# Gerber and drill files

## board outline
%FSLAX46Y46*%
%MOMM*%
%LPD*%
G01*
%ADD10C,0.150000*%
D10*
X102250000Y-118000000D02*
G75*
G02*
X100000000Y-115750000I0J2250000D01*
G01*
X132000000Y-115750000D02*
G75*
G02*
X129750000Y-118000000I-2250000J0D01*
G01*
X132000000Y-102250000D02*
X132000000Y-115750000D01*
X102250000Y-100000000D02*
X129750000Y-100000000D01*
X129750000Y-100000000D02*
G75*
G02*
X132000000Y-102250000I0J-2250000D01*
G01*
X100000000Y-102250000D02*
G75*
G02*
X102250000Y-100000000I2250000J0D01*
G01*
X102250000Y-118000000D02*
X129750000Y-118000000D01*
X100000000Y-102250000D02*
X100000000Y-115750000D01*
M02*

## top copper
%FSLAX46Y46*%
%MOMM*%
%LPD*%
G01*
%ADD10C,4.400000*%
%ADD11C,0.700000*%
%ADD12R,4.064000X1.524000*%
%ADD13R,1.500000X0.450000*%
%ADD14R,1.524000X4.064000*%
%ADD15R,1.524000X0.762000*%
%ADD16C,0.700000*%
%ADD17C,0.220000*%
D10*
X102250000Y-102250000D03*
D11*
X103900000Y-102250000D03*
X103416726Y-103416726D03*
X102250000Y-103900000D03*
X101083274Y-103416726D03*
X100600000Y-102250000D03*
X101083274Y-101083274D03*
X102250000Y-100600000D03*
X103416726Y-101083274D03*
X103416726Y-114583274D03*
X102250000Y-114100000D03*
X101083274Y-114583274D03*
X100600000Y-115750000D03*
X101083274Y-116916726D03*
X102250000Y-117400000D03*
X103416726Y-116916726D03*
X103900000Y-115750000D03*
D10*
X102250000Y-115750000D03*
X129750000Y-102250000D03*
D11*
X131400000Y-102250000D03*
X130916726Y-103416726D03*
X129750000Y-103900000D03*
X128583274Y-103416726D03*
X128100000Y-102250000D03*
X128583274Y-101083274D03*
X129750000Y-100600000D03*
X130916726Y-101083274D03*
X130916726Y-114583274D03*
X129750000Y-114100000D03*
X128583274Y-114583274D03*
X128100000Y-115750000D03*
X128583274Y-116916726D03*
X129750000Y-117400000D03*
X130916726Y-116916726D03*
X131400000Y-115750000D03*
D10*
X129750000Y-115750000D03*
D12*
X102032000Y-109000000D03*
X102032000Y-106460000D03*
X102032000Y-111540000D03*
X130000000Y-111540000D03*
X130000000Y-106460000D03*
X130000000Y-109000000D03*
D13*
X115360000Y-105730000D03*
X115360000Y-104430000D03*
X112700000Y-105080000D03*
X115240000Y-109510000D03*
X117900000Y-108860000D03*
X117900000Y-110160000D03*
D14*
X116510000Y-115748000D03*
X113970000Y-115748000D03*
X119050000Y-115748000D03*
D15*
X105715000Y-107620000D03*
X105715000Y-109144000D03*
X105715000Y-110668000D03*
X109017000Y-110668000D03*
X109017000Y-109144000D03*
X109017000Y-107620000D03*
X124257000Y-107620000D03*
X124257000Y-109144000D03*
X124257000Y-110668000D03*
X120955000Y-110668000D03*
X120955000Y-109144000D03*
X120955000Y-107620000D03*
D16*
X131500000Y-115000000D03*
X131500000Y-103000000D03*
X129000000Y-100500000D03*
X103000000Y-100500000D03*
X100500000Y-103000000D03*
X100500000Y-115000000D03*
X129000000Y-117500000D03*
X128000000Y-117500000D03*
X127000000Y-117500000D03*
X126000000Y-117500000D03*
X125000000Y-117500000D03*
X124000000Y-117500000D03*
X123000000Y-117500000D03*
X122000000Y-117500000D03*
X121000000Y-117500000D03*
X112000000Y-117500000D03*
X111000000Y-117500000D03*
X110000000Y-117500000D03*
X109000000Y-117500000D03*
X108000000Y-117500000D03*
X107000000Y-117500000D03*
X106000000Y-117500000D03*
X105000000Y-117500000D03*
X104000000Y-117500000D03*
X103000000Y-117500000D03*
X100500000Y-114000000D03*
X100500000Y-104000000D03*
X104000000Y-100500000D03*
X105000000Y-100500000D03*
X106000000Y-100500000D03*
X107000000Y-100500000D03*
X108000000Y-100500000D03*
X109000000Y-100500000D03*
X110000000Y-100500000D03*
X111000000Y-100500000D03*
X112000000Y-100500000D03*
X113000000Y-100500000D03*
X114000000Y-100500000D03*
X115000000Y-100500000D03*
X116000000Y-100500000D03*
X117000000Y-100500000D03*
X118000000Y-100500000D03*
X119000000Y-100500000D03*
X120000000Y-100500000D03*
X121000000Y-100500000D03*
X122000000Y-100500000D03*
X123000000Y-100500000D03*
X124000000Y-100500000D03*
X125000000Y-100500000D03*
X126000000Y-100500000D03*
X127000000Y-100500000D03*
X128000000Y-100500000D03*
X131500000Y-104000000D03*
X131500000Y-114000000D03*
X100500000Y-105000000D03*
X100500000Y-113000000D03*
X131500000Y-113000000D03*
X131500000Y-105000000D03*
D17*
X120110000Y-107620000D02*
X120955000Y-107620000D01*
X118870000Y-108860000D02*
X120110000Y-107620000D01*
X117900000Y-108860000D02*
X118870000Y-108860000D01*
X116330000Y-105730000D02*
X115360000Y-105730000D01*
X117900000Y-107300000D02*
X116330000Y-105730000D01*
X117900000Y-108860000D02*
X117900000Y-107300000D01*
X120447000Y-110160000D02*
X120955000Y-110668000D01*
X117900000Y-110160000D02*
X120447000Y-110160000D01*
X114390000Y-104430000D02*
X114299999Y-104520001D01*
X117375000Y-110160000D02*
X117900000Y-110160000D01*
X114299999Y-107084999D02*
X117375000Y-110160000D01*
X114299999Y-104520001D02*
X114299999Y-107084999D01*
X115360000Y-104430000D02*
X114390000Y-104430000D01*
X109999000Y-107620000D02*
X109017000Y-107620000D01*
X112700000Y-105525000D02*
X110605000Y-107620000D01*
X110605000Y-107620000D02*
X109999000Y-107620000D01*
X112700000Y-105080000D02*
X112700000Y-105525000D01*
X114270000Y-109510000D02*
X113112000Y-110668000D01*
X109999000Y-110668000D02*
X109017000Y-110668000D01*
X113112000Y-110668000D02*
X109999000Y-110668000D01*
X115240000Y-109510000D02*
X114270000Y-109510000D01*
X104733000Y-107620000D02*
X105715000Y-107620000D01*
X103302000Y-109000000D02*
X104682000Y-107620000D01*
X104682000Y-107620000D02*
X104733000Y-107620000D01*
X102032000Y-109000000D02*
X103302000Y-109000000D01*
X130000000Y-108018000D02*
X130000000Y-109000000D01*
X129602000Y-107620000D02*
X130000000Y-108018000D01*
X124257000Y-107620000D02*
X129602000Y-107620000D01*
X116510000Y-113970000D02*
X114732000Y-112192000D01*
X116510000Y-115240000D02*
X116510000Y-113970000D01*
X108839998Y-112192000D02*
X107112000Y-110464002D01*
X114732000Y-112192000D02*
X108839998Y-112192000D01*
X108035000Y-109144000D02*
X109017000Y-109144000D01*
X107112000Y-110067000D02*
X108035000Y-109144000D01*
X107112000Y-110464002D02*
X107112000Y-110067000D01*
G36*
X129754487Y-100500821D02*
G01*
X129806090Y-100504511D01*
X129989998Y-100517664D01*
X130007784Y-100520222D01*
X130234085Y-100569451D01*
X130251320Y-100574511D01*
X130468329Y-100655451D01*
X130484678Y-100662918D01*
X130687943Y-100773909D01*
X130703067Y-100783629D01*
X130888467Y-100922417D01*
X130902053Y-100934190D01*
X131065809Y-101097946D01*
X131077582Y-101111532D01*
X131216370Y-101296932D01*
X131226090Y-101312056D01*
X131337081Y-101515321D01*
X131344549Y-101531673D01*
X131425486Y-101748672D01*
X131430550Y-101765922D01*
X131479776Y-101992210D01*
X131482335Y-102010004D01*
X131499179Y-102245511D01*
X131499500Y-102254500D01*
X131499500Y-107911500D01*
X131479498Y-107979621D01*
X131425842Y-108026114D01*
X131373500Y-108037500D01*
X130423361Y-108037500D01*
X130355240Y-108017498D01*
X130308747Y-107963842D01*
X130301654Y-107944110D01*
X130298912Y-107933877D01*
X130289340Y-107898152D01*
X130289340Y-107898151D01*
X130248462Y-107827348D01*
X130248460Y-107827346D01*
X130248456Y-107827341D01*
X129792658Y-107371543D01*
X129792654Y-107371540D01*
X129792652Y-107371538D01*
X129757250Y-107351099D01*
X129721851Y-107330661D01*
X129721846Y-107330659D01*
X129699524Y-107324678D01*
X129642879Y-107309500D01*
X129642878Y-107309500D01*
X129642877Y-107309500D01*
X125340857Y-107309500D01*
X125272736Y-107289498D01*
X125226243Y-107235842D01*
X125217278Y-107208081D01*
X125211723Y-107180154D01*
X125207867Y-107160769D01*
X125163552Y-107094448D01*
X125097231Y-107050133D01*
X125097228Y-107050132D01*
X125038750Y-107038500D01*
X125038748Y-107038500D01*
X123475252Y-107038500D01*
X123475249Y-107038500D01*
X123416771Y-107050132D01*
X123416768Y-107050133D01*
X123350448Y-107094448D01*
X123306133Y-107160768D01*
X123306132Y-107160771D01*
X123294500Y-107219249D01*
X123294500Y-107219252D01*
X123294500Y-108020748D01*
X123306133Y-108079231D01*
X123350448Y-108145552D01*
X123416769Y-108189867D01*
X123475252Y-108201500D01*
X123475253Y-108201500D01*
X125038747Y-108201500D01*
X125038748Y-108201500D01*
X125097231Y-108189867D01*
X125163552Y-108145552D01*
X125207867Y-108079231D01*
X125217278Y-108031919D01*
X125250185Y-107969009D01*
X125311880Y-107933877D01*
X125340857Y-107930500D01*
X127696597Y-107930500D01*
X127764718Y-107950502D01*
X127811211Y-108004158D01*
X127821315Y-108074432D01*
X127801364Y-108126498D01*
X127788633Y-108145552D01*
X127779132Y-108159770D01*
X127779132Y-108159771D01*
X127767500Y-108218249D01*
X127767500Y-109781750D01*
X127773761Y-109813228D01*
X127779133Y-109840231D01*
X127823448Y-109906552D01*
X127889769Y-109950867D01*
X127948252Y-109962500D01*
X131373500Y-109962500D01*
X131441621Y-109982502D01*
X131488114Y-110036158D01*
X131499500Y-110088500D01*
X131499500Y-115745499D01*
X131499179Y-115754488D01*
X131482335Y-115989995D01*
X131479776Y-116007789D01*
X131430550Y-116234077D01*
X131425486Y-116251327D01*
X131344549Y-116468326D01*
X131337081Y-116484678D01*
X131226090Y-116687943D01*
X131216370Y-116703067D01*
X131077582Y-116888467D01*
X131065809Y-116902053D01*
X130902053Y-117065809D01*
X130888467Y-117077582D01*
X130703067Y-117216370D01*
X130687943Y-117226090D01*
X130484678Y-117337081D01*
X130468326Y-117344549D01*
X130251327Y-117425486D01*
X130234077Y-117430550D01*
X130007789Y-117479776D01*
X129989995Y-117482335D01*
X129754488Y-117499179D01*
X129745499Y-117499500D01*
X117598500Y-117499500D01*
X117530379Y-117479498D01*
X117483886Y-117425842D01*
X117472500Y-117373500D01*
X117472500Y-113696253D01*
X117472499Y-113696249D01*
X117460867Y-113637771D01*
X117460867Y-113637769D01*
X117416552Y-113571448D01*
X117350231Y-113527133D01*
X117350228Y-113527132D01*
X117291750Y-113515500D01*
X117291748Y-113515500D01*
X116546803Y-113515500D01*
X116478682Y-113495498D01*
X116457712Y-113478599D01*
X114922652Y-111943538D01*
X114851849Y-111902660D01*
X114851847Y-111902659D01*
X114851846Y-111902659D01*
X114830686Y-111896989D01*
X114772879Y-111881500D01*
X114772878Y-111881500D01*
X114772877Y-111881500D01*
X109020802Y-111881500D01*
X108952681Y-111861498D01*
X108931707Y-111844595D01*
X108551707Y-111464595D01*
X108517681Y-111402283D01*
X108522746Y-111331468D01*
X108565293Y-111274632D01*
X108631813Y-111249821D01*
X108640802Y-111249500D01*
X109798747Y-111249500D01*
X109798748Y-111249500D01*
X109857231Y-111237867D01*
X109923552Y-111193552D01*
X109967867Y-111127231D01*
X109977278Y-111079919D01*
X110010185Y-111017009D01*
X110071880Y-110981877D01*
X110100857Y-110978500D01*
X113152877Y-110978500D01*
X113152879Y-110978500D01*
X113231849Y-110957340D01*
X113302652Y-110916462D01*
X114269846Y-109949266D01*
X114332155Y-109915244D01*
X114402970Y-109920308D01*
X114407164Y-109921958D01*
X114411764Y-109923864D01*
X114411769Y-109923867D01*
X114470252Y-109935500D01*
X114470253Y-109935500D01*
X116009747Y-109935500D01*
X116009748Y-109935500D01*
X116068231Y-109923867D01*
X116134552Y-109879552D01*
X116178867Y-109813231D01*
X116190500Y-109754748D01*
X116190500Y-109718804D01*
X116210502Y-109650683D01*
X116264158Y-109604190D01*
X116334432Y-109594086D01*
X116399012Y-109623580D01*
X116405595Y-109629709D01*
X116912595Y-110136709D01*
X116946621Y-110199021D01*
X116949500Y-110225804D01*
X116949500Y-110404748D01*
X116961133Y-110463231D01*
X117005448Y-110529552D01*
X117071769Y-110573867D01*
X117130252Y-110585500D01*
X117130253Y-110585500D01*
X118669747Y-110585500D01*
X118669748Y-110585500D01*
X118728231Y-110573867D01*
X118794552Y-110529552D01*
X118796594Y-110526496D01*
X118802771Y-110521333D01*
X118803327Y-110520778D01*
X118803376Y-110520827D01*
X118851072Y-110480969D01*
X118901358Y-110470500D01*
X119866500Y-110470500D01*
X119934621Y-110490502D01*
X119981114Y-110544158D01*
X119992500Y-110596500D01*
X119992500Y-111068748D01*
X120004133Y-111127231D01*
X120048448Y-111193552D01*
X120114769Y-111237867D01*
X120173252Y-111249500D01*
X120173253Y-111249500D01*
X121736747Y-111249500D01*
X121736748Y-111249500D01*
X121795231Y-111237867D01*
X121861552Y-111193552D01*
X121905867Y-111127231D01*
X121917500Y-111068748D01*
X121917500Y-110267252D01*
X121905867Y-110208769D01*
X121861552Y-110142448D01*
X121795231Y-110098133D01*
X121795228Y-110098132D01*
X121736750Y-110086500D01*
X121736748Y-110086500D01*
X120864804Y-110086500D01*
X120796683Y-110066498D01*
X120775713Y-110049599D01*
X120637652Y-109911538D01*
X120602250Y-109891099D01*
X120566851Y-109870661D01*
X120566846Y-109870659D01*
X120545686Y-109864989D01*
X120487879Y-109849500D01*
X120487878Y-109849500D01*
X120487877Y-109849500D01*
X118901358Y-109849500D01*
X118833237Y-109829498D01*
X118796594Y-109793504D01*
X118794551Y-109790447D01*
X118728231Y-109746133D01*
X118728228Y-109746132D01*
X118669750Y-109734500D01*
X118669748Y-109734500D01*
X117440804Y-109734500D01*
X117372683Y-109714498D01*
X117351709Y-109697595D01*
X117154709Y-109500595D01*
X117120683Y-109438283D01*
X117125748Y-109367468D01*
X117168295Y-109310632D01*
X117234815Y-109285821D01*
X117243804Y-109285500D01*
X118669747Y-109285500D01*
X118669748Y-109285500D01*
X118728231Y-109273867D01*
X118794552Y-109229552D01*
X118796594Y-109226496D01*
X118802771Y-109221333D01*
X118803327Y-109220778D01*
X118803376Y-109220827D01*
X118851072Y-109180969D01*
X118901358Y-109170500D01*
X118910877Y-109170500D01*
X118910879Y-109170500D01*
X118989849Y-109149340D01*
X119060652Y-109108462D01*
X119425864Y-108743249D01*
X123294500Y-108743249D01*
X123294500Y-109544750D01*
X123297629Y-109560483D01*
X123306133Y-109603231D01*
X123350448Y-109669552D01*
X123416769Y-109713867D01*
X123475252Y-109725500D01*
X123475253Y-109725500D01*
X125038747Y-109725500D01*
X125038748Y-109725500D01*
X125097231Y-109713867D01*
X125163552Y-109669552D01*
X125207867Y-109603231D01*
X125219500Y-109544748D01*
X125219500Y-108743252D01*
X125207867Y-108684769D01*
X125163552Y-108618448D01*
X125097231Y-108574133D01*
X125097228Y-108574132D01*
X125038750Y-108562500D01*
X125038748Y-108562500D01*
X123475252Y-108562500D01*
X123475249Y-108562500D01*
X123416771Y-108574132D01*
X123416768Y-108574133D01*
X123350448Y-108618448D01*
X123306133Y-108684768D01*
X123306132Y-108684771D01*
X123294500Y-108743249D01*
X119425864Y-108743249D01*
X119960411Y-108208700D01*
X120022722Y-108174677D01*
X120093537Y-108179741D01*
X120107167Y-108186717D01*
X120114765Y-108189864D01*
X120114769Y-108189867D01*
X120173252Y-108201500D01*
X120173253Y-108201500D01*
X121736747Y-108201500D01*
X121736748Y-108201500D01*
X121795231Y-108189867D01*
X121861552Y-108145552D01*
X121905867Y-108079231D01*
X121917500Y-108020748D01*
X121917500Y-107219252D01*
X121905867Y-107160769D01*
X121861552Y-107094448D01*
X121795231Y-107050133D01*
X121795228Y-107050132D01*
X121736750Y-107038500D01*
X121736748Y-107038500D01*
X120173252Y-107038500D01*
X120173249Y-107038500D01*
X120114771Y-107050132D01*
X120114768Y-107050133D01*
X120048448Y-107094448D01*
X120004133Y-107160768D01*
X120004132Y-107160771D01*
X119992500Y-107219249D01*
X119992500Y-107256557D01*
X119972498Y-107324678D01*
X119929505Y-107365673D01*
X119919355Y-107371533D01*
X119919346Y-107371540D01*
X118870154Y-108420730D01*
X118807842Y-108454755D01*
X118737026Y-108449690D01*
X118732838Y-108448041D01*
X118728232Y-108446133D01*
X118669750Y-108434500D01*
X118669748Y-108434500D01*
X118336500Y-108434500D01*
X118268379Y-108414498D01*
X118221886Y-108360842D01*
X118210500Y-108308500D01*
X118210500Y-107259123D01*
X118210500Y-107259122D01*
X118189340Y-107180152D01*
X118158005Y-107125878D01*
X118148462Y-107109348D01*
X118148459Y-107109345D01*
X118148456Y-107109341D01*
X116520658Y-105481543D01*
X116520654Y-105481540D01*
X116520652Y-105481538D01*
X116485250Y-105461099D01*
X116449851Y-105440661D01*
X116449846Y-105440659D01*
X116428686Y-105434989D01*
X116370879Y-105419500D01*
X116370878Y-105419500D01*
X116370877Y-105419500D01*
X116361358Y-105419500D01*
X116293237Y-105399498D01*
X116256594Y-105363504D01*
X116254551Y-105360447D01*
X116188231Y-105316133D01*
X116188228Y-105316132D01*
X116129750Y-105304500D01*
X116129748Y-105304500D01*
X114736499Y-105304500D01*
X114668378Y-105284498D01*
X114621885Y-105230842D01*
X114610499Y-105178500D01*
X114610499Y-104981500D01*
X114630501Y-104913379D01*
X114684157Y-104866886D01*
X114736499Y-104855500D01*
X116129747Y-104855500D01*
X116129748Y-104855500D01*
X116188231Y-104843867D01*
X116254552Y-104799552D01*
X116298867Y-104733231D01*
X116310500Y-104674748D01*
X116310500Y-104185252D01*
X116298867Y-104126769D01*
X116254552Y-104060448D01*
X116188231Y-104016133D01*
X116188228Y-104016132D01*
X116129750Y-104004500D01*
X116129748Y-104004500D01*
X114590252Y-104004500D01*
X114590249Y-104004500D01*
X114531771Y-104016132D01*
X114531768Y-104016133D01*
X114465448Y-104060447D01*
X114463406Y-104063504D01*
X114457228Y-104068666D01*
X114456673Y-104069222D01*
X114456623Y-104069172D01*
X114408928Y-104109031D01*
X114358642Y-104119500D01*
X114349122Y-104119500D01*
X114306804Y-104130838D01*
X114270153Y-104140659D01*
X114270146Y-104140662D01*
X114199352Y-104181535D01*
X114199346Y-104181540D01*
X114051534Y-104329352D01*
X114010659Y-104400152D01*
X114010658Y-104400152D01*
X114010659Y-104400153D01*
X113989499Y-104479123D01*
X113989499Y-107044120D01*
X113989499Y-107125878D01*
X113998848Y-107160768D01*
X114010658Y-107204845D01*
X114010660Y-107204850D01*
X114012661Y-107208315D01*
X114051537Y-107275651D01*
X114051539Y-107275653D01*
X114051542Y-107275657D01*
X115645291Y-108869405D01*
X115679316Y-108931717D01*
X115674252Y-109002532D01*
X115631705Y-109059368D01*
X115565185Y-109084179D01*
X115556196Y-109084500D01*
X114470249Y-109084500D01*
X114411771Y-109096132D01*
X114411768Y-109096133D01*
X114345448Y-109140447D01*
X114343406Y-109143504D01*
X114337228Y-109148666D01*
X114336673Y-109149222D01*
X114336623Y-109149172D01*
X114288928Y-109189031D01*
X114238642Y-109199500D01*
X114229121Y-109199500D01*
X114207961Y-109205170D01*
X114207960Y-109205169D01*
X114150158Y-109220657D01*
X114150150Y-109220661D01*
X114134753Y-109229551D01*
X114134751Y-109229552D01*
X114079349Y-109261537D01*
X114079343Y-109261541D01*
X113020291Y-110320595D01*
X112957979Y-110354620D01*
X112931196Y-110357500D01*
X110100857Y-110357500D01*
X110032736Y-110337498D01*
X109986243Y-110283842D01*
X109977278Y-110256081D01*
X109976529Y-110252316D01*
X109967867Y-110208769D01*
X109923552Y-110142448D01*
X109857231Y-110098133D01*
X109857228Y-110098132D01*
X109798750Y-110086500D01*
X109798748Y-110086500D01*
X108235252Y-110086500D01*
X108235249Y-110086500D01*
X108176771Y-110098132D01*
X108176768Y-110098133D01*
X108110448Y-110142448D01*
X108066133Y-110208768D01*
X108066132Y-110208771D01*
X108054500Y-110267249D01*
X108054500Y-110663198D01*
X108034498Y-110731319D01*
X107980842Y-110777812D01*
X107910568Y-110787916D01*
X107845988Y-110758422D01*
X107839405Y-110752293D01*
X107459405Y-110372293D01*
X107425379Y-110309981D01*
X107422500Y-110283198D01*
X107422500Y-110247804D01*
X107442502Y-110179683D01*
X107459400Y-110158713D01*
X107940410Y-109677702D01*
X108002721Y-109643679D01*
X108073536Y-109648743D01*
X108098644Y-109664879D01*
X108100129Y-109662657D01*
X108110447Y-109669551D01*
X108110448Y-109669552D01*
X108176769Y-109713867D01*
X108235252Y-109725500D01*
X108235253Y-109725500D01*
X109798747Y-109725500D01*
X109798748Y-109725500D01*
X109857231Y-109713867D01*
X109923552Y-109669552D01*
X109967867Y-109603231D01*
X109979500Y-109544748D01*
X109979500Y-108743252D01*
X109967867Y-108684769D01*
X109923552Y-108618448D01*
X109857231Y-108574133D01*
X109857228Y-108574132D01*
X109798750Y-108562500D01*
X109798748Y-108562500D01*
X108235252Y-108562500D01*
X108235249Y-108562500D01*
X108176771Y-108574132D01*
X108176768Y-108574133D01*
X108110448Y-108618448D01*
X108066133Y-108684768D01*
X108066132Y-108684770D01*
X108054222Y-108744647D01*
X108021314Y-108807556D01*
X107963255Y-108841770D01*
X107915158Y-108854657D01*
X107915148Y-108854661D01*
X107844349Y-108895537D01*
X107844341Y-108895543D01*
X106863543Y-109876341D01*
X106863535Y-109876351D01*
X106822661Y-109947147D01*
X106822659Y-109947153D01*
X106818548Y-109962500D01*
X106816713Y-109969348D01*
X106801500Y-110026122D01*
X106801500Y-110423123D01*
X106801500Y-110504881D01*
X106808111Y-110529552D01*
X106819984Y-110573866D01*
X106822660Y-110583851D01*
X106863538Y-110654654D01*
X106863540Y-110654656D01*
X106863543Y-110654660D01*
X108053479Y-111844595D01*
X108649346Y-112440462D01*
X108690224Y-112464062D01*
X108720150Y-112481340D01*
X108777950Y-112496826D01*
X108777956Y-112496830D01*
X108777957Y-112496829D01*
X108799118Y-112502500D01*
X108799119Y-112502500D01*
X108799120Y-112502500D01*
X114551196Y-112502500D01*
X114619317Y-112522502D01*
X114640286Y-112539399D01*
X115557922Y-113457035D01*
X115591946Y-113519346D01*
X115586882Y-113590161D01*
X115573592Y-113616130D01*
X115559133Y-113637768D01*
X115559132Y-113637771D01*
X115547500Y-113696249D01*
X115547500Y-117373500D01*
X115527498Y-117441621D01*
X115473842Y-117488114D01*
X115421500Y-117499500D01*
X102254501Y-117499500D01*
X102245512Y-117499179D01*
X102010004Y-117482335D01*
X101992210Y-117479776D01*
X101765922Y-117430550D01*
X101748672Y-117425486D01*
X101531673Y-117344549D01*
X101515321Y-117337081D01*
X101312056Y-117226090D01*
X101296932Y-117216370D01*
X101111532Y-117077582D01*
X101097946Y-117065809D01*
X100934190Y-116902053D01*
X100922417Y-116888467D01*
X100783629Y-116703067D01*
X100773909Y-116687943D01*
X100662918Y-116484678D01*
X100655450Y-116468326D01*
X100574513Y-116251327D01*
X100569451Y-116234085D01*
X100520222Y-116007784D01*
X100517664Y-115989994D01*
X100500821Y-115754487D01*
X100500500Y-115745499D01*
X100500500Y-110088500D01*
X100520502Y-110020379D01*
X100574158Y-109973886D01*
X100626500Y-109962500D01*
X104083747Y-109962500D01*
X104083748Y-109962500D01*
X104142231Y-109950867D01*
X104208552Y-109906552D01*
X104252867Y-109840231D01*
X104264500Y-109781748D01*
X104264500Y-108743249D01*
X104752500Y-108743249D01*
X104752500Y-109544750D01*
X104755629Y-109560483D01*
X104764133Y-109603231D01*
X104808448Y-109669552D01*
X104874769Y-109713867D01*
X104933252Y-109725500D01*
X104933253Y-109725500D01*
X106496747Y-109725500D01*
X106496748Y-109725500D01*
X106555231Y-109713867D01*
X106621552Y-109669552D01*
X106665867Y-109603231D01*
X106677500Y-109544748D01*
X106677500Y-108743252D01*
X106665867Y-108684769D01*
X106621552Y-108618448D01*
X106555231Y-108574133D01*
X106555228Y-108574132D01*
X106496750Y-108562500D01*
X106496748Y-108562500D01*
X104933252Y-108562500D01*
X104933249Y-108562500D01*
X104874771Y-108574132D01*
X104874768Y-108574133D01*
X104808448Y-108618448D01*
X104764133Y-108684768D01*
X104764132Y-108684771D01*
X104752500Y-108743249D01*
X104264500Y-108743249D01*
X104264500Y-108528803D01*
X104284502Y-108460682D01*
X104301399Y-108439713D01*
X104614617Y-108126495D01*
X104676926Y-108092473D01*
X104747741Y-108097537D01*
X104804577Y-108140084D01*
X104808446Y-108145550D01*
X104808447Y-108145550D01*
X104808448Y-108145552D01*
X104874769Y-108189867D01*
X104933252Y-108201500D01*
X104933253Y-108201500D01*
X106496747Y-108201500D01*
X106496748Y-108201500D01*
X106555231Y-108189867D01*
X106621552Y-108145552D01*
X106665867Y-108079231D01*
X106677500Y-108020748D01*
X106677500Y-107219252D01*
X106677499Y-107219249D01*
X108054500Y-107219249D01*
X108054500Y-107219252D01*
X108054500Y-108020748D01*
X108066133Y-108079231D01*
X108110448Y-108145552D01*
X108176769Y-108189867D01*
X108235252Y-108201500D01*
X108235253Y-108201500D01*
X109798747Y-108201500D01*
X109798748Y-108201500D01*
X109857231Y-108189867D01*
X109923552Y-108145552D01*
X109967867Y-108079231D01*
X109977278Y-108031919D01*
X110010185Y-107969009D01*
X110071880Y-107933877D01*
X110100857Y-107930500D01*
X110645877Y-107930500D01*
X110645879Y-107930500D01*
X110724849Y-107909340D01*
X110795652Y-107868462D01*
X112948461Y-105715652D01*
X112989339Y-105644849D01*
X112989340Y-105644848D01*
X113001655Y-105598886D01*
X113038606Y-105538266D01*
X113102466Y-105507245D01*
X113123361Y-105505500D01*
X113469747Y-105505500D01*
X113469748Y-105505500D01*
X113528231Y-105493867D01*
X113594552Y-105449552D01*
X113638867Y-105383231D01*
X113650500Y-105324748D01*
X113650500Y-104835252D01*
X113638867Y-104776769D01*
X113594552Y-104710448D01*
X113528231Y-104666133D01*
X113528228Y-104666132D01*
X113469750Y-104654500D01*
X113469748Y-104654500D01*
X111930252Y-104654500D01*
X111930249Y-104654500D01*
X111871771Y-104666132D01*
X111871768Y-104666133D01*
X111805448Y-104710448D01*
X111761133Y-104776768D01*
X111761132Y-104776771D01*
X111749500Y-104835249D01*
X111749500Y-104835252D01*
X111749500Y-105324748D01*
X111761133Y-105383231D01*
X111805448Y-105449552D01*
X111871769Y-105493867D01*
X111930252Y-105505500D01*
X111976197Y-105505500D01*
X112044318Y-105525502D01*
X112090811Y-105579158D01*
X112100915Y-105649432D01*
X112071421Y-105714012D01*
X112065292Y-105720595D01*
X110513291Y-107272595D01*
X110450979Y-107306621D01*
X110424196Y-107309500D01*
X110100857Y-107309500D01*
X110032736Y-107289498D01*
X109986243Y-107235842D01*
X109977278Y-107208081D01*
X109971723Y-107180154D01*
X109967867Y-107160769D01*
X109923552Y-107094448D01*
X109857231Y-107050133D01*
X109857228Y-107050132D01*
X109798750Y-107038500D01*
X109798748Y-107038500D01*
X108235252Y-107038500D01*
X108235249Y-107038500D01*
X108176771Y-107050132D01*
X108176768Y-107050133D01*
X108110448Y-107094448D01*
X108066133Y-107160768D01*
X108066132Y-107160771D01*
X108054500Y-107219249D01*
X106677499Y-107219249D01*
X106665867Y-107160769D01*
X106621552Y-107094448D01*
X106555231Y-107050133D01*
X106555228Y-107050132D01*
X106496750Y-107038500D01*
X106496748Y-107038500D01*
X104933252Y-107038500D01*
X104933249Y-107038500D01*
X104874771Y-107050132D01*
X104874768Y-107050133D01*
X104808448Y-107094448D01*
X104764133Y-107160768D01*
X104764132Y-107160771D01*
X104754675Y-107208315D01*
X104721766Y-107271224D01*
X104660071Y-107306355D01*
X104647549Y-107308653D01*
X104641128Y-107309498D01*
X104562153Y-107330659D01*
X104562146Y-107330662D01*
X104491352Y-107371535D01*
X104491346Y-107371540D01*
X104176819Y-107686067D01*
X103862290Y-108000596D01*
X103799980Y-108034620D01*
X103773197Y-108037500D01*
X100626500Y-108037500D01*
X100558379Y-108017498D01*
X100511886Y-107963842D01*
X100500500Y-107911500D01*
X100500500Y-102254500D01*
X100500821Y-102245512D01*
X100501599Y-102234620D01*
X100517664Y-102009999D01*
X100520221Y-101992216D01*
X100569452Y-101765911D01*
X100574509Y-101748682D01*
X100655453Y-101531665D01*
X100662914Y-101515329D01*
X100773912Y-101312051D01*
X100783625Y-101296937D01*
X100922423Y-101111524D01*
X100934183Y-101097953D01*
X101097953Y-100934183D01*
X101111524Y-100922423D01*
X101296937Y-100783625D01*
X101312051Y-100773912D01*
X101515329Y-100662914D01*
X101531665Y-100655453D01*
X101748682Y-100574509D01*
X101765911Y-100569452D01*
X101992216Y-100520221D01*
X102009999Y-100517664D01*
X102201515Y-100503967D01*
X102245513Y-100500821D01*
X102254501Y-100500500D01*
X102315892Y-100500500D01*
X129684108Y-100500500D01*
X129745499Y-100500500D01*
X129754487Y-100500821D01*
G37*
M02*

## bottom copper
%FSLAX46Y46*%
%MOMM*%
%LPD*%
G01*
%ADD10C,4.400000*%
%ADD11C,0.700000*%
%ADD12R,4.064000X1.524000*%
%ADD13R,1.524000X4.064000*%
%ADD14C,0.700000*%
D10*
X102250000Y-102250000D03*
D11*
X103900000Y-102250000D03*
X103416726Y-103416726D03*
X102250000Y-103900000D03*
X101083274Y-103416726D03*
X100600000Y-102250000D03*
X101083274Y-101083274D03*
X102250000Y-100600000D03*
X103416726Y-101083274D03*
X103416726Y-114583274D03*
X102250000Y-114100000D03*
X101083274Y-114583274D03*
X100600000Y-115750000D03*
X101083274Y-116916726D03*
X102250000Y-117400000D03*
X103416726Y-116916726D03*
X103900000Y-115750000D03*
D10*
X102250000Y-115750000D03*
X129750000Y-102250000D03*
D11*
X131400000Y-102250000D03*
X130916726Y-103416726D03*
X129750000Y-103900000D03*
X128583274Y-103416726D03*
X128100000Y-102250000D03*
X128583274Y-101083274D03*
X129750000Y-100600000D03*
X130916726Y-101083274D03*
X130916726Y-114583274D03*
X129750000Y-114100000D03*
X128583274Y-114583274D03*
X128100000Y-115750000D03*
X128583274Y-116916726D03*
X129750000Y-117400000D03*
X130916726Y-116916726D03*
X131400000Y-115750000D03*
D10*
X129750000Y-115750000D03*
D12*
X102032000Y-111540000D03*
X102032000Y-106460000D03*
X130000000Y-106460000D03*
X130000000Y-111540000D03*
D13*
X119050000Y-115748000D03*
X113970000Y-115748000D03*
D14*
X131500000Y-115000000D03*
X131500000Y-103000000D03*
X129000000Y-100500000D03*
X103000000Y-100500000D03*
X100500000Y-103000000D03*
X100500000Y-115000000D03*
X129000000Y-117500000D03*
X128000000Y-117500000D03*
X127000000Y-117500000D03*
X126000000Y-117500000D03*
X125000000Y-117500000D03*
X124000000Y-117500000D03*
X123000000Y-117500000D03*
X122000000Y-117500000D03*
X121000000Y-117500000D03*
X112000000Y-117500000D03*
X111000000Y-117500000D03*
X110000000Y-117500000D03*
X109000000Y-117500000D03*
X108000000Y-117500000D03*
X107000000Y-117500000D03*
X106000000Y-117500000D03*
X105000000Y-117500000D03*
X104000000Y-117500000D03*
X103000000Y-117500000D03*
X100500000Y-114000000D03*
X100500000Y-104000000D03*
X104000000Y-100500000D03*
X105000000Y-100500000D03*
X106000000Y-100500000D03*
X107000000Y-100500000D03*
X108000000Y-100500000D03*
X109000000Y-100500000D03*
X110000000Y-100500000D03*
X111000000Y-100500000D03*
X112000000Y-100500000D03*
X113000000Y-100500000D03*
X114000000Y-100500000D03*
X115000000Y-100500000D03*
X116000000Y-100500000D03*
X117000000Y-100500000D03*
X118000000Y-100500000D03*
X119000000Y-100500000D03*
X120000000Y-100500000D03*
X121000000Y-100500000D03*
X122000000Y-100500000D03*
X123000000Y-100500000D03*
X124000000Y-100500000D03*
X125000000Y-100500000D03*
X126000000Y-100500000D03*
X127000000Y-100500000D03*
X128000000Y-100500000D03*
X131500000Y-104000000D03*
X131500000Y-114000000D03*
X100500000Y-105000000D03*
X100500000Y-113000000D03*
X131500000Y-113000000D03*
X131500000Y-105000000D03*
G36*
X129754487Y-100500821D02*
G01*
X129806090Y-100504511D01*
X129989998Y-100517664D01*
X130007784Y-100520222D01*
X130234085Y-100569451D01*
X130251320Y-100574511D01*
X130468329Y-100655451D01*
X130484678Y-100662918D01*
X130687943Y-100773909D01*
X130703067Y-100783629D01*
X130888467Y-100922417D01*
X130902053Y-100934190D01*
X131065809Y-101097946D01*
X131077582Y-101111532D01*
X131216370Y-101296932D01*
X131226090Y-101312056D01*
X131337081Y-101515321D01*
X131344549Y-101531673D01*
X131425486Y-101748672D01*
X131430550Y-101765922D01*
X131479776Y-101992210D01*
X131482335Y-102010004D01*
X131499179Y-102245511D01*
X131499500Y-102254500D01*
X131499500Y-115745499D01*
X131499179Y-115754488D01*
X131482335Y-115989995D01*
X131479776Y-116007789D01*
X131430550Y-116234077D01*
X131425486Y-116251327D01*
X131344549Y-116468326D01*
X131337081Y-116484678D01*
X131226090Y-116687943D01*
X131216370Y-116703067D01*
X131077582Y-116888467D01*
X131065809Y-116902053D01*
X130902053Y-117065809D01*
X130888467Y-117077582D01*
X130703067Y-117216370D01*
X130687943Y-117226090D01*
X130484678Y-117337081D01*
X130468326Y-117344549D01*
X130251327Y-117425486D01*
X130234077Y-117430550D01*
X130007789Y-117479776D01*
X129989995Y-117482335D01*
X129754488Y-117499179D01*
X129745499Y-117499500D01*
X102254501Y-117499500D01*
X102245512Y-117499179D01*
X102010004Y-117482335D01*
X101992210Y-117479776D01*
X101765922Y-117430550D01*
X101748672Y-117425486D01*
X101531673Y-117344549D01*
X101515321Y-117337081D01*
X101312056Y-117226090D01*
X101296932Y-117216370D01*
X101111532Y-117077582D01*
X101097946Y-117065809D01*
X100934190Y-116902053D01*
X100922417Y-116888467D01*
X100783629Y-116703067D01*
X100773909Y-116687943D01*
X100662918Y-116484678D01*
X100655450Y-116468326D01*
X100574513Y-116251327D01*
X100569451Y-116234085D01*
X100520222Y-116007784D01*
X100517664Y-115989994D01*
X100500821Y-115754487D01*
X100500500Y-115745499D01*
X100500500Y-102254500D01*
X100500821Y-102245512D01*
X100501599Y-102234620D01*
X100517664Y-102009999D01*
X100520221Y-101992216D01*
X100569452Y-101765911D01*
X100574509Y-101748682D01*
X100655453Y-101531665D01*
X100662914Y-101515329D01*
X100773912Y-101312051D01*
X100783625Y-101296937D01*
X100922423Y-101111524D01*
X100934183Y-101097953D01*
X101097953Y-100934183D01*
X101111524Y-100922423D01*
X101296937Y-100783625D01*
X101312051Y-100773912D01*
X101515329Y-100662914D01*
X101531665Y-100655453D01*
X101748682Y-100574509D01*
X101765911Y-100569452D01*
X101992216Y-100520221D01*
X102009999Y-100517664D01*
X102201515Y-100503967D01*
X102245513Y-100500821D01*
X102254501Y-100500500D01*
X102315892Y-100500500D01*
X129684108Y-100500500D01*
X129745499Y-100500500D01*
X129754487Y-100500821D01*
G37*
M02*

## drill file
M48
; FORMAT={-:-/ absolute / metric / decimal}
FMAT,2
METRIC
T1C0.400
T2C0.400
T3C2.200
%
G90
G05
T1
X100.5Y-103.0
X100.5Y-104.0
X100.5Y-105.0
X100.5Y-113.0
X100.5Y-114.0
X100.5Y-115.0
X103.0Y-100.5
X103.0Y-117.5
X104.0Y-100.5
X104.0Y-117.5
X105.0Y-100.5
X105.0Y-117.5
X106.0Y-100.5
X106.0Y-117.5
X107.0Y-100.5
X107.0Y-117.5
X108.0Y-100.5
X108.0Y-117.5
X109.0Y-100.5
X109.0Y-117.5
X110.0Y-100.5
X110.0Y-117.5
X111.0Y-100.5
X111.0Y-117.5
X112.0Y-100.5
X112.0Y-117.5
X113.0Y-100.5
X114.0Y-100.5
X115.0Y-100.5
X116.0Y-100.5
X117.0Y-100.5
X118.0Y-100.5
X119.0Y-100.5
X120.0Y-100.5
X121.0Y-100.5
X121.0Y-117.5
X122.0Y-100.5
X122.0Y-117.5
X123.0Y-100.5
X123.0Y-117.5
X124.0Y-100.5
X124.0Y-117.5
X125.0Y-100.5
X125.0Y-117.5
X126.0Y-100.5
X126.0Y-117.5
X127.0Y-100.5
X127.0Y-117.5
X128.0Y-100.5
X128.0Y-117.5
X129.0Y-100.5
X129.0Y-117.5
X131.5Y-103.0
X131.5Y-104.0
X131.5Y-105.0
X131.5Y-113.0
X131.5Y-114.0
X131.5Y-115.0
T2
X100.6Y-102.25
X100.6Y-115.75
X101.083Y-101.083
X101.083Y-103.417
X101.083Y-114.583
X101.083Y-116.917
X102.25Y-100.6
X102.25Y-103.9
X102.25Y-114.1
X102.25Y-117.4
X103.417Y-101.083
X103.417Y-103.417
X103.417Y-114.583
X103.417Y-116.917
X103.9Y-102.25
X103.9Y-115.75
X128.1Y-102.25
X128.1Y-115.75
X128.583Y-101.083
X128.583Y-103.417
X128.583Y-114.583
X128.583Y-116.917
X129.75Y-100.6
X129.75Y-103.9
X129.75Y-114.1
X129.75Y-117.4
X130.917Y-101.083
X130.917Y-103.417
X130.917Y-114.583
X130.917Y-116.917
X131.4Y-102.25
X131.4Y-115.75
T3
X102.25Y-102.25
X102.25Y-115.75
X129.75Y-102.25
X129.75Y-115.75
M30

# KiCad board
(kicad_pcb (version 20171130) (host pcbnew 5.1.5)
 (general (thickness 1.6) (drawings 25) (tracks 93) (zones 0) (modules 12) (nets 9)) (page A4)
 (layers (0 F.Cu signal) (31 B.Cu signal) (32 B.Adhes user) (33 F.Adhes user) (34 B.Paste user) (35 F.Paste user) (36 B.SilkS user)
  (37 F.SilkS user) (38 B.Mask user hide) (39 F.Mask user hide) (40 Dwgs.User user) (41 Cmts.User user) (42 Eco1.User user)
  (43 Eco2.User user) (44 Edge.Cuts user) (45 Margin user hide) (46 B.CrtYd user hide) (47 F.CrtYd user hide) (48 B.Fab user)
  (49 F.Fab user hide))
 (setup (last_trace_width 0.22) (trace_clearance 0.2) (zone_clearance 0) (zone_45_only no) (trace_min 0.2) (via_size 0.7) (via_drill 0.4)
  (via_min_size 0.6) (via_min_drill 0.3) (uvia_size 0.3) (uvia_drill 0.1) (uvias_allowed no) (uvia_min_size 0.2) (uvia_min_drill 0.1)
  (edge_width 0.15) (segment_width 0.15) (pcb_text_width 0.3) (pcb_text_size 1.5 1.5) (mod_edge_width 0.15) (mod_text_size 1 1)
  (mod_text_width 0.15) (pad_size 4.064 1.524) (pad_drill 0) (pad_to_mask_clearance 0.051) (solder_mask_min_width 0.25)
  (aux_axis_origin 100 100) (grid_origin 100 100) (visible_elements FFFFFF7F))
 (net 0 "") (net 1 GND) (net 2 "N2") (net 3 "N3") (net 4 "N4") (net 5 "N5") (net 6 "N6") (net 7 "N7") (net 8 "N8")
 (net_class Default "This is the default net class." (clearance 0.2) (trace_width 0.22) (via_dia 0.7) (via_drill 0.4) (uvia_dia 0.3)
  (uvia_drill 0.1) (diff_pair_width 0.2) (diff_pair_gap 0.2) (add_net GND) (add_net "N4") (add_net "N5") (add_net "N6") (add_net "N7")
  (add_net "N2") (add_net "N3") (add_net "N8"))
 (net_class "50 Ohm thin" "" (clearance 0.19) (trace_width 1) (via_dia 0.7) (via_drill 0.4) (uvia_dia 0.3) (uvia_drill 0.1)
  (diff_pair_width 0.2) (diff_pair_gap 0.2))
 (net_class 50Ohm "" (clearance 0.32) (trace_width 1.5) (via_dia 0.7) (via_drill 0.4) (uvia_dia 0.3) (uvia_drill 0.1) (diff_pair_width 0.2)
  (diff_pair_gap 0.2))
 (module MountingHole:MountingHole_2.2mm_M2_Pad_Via (layer F.Cu) (at 102.25 102.25)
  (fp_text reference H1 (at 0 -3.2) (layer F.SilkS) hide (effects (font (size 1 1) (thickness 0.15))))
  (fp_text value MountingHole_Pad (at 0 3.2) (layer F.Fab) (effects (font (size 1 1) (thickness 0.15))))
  (pad 1 thru_hole circle (at 0 0) (size 4.4 4.4) (drill 2.2) (layers *.Cu *.Mask) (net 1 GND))
  (pad 1 thru_hole circle (at 1.65 0) (size 0.7 0.7) (drill 0.4) (layers *.Cu *.Mask) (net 1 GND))
  (pad 1 thru_hole circle (at 1.166726 1.166726) (size 0.7 0.7) (drill 0.4) (layers *.Cu *.Mask) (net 1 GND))
  (pad 1 thru_hole circle (at 0 1.65) (size 0.7 0.7) (drill 0.4) (layers *.Cu *.Mask) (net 1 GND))
  (pad 1 thru_hole circle (at -1.166726 1.166726) (size 0.7 0.7) (drill 0.4) (layers *.Cu *.Mask) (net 1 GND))
  (pad 1 thru_hole circle (at -1.65 0) (size 0.7 0.7) (drill 0.4) (layers *.Cu *.Mask) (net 1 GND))
  (pad 1 thru_hole circle (at -1.166726 -1.166726) (size 0.7 0.7) (drill 0.4) (layers *.Cu *.Mask) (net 1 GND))
  (pad 1 thru_hole circle (at 0 -1.65) (size 0.7 0.7) (drill 0.4) (layers *.Cu *.Mask) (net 1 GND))
  (pad 1 thru_hole circle (at 1.166726 -1.166726) (size 0.7 0.7) (drill 0.4) (layers *.Cu *.Mask) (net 1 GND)))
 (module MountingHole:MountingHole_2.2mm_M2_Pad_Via (layer F.Cu) (at 102.25 115.75)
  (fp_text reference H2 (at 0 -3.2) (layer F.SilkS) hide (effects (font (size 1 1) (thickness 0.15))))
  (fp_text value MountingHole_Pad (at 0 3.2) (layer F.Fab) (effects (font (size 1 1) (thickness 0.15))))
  (pad 1 thru_hole circle (at 1.166726 -1.166726) (size 0.7 0.7) (drill 0.4) (layers *.Cu *.Mask) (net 1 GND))
  (pad 1 thru_hole circle (at 0 -1.65) (size 0.7 0.7) (drill 0.4) (layers *.Cu *.Mask) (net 1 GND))
  (pad 1 thru_hole circle (at -1.166726 -1.166726) (size 0.7 0.7) (drill 0.4) (layers *.Cu *.Mask) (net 1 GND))
  (pad 1 thru_hole circle (at -1.65 0) (size 0.7 0.7) (drill 0.4) (layers *.Cu *.Mask) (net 1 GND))
  (pad 1 thru_hole circle (at -1.166726 1.166726) (size 0.7 0.7) (drill 0.4) (layers *.Cu *.Mask) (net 1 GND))
  (pad 1 thru_hole circle (at 0 1.65) (size 0.7 0.7) (drill 0.4) (layers *.Cu *.Mask) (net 1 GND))
  (pad 1 thru_hole circle (at 1.166726 1.166726) (size 0.7 0.7) (drill 0.4) (layers *.Cu *.Mask) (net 1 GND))
  (pad 1 thru_hole circle (at 1.65 0) (size 0.7 0.7) (drill 0.4) (layers *.Cu *.Mask) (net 1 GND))
  (pad 1 thru_hole circle (at 0 0) (size 4.4 4.4) (drill 2.2) (layers *.Cu *.Mask) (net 1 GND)))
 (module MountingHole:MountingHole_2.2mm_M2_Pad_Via (layer F.Cu) (at 129.75 102.25)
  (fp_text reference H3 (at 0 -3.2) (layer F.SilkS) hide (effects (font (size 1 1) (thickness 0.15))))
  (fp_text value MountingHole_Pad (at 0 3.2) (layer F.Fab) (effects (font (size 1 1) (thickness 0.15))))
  (pad 1 thru_hole circle (at 0 0) (size 4.4 4.4) (drill 2.2) (layers *.Cu *.Mask) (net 1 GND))
  (pad 1 thru_hole circle (at 1.65 0) (size 0.7 0.7) (drill 0.4) (layers *.Cu *.Mask) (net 1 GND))
  (pad 1 thru_hole circle (at 1.166726 1.166726) (size 0.7 0.7) (drill 0.4) (layers *.Cu *.Mask) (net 1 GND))
  (pad 1 thru_hole circle (at 0 1.65) (size 0.7 0.7) (drill 0.4) (layers *.Cu *.Mask) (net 1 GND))
  (pad 1 thru_hole circle (at -1.166726 1.166726) (size 0.7 0.7) (drill 0.4) (layers *.Cu *.Mask) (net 1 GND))
  (pad 1 thru_hole circle (at -1.65 0) (size 0.7 0.7) (drill 0.4) (layers *.Cu *.Mask) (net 1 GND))
  (pad 1 thru_hole circle (at -1.166726 -1.166726) (size 0.7 0.7) (drill 0.4) (layers *.Cu *.Mask) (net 1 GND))
  (pad 1 thru_hole circle (at 0 -1.65) (size 0.7 0.7) (drill 0.4) (layers *.Cu *.Mask) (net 1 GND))
  (pad 1 thru_hole circle (at 1.166726 -1.166726) (size 0.7 0.7) (drill 0.4) (layers *.Cu *.Mask) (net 1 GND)))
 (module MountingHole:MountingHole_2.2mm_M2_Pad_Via (layer F.Cu) (at 129.75 115.75)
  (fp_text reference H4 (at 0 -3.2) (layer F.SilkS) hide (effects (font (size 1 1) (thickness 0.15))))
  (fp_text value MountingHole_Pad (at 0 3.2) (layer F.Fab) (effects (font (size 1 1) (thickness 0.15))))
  (pad 1 thru_hole circle (at 1.166726 -1.166726) (size 0.7 0.7) (drill 0.4) (layers *.Cu *.Mask) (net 1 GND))
  (pad 1 thru_hole circle (at 0 -1.65) (size 0.7 0.7) (drill 0.4) (layers *.Cu *.Mask) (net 1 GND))
  (pad 1 thru_hole circle (at -1.166726 -1.166726) (size 0.7 0.7) (drill 0.4) (layers *.Cu *.Mask) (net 1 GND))
  (pad 1 thru_hole circle (at -1.65 0) (size 0.7 0.7) (drill 0.4) (layers *.Cu *.Mask) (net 1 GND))
  (pad 1 thru_hole circle (at -1.166726 1.166726) (size 0.7 0.7) (drill 0.4) (layers *.Cu *.Mask) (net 1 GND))
  (pad 1 thru_hole circle (at 0 1.65) (size 0.7 0.7) (drill 0.4) (layers *.Cu *.Mask) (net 1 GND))
  (pad 1 thru_hole circle (at 1.166726 1.166726) (size 0.7 0.7) (drill 0.4) (layers *.Cu *.Mask) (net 1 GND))
  (pad 1 thru_hole circle (at 1.65 0) (size 0.7 0.7) (drill 0.4) (layers *.Cu *.Mask) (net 1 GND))
  (pad 1 thru_hole circle (at 0 0) (size 4.4 4.4) (drill 2.2) (layers *.Cu *.Mask) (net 1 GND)))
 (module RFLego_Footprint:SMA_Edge (layer F.Cu) (at 100 109)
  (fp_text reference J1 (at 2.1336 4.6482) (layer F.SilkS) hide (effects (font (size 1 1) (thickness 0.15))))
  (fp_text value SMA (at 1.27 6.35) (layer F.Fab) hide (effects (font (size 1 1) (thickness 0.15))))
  (pad 1 smd rect (at 2.032 0) (size 4.064 1.524) (layers F.Cu F.Mask) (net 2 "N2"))
  (pad 2 smd rect (at 2.032 -2.54) (size 4.064 1.524) (layers F.Cu F.Mask) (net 1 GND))
  (pad 2 smd rect (at 2.032 2.54) (size 4.064 1.524) (layers B.Cu B.Mask) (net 1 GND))
  (pad 2 smd rect (at 2.032 -2.54) (size 4.064 1.524) (layers B.Cu B.Mask) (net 1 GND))
  (pad 2 smd rect (at 2.032 2.54) (size 4.064 1.524) (layers F.Cu F.Mask) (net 1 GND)))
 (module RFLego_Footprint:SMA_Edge (layer F.Cu) (at 127.968 109)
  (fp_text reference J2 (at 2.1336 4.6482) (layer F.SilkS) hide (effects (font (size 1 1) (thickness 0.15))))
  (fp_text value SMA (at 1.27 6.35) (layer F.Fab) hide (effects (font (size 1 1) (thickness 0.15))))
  (pad 2 smd rect (at 2.032 2.54) (size 4.064 1.524) (layers F.Cu F.Mask) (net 1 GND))
  (pad 2 smd rect (at 2.032 -2.54) (size 4.064 1.524) (layers B.Cu B.Mask) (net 1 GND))
  (pad 2 smd rect (at 2.032 2.54) (size 4.064 1.524) (layers B.Cu B.Mask) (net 1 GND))
  (pad 2 smd rect (at 2.032 -2.54) (size 4.064 1.524) (layers F.Cu F.Mask) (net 1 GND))
  (pad 1 smd rect (at 2.032 0) (size 4.064 1.524) (layers F.Cu F.Mask) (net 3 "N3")))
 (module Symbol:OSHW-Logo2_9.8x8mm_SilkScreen (layer B.Cu) (at 109.5 113.25 180)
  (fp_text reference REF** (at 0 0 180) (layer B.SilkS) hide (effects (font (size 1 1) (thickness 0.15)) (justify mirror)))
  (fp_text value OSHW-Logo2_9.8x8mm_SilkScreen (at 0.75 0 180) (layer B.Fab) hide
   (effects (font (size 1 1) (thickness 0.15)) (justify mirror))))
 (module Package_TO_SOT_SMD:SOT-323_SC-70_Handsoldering (layer F.Cu) (at 114.03 105.08 180)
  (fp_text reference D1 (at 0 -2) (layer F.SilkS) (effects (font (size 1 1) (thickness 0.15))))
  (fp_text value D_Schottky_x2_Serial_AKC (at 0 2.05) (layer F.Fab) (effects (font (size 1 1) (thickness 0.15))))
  (pad 1 smd rect (at -1.33 -0.65 90) (size 0.45 1.5) (layers F.Cu F.Paste F.Mask) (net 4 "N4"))
  (pad 2 smd rect (at -1.33 0.65 90) (size 0.45 1.5) (layers F.Cu F.Paste F.Mask) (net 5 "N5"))
  (pad 3 smd rect (at 1.33 0 90) (size 0.45 1.5) (layers F.Cu F.Paste F.Mask) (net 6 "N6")))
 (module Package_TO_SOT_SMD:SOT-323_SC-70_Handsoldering (layer F.Cu) (at 116.57 109.51 180)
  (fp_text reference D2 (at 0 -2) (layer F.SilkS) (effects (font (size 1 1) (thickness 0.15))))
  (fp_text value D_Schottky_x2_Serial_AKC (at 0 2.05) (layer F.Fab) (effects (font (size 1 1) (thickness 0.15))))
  (pad 3 smd rect (at 1.33 0 90) (size 0.45 1.5) (layers F.Cu F.Paste F.Mask) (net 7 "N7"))
  (pad 2 smd rect (at -1.33 0.65 90) (size 0.45 1.5) (layers F.Cu F.Paste F.Mask) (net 4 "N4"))
  (pad 1 smd rect (at -1.33 -0.65 90) (size 0.45 1.5) (layers F.Cu F.Paste F.Mask) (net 5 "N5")))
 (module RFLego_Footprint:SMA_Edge (layer F.Cu) (at 116.51 117.78 90)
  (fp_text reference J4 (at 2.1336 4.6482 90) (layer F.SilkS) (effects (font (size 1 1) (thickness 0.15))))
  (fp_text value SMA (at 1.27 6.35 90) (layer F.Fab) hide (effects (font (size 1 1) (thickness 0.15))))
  (pad 1 smd rect (at 2.032 0 90) (size 4.064 1.524) (layers F.Cu F.Mask) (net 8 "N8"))
  (pad 2 smd rect (at 2.032 -2.54 90) (size 4.064 1.524) (layers F.Cu F.Mask) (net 1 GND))
  (pad 2 smd rect (at 2.032 2.54 90) (size 4.064 1.524) (layers B.Cu B.Mask) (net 1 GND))
  (pad 2 smd rect (at 2.032 -2.54 90) (size 4.064 1.524) (layers B.Cu B.Mask) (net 1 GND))
  (pad 2 smd rect (at 2.032 2.54 90) (size 4.064 1.524) (layers F.Cu F.Mask) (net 1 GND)))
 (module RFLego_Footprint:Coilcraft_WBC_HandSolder (layer F.Cu) (at 108.89 107.62 270)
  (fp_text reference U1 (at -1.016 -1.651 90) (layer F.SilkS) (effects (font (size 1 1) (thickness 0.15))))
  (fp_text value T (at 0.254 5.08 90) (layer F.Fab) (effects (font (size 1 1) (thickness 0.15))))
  (pad 6 smd rect (at 0 3.175 270) (size 0.762 1.524) (layers F.Cu F.Paste F.Mask) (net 2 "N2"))
  (pad 5 smd rect (at 1.524 3.175 270) (size 0.762 1.524) (layers F.Cu F.Paste F.Mask))
  (pad 4 smd rect (at 3.048 3.175 270) (size 0.762 1.524) (layers F.Cu F.Paste F.Mask) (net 1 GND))
  (pad 3 smd rect (at 3.048 -0.127 270) (size 0.762 1.524) (layers F.Cu F.Paste F.Mask) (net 7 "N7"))
  (pad 2 smd rect (at 1.524 -0.127 270) (size 0.762 1.524) (layers F.Cu F.Paste F.Mask) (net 8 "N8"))
  (pad 1 smd rect (at 0 -0.127 270) (size 0.762 1.524) (layers F.Cu F.Paste F.Mask) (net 6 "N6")))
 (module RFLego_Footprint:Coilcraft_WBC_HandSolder (layer F.Cu) (at 124.13 107.62 270)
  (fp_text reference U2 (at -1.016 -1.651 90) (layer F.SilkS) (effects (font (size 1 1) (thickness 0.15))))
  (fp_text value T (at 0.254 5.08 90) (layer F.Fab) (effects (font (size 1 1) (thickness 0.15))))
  (pad 1 smd rect (at 0 -0.127 270) (size 0.762 1.524) (layers F.Cu F.Paste F.Mask) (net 3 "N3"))
  (pad 2 smd rect (at 1.524 -0.127 270) (size 0.762 1.524) (layers F.Cu F.Paste F.Mask))
  (pad 3 smd rect (at 3.048 -0.127 270) (size 0.762 1.524) (layers F.Cu F.Paste F.Mask) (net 1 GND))
  (pad 4 smd rect (at 3.048 3.175 270) (size 0.762 1.524) (layers F.Cu F.Paste F.Mask) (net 5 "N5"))
  (pad 5 smd rect (at 1.524 3.175 270) (size 0.762 1.524) (layers F.Cu F.Paste F.Mask) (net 1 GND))
  (pad 6 smd rect (at 0 3.175 270) (size 0.762 1.524) (layers F.Cu F.Paste F.Mask) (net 4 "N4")))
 (gr_arc (start 102.25 115.75) (end 100 115.75) (angle -90) (layer Edge.Cuts) (width 0.15))
 (gr_arc (start 129.75 115.75) (end 129.75 118) (angle -90) (layer Edge.Cuts) (width 0.15))
 (gr_line (start 132 102.25) (end 132 115.75) (layer Edge.Cuts) (width 0.15))
 (gr_line (start 102.25 100) (end 129.75 100) (layer Edge.Cuts) (width 0.15))
 (gr_arc (start 129.75 102.25) (end 132 102.25) (angle -90) (layer Edge.Cuts) (width 0.15))
 (gr_arc (start 102.25 102.25) (end 102.25 100) (angle -90) (layer Edge.Cuts) (width 0.15))
 (gr_line (start 102.25 118) (end 129.75 118) (layer Edge.Cuts) (width 0.15))
 (gr_line (start 100 102.25) (end 100 115.75) (layer Edge.Cuts) (width 0.15))
 (via (at 131.5 115) (size 0.7) (drill 0.4) (layers F.Cu B.Cu) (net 1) (status 30))
 (via (at 131.5 103) (size 0.7) (drill 0.4) (layers F.Cu B.Cu) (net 1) (status 30))
 (via (at 129 100.5) (size 0.7) (drill 0.4) (layers F.Cu B.Cu) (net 1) (status 30))
 (via (at 103 100.5) (size 0.7) (drill 0.4) (layers F.Cu B.Cu) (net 1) (status 30))
 (via (at 100.5 103) (size 0.7) (drill 0.4) (layers F.Cu B.Cu) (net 1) (status 30))
 (via (at 100.5 115) (size 0.7) (drill 0.4) (layers F.Cu B.Cu) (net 1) (status 30))
 (via (at 129 117.5) (size 0.7) (drill 0.4) (layers F.Cu B.Cu) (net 1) (status 30))
 (via (at 128 117.5) (size 0.7) (drill 0.4) (layers F.Cu B.Cu) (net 1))
 (via (at 127 117.5) (size 0.7) (drill 0.4) (layers F.Cu B.Cu) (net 1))
 (via (at 126 117.5) (size 0.7) (drill 0.4) (layers F.Cu B.Cu) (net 1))
 (via (at 125 117.5) (size 0.7) (drill 0.4) (layers F.Cu B.Cu) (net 1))
 (via (at 124 117.5) (size 0.7) (drill 0.4) (layers F.Cu B.Cu) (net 1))
 (via (at 123 117.5) (size 0.7) (drill 0.4) (layers F.Cu B.Cu) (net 1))
 (via (at 122 117.5) (size 0.7) (drill 0.4) (layers F.Cu B.Cu) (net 1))
 (via (at 121 117.5) (size 0.7) (drill 0.4) (layers F.Cu B.Cu) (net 1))
 (via (at 112 117.5) (size 0.7) (drill 0.4) (layers F.Cu B.Cu) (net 1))
 (via (at 111 117.5) (size 0.7) (drill 0.4) (layers F.Cu B.Cu) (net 1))
 (via (at 110 117.5) (size 0.7) (drill 0.4) (layers F.Cu B.Cu) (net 1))
 (via (at 109 117.5) (size 0.7) (drill 0.4) (layers F.Cu B.Cu) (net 1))
 (via (at 108 117.5) (size 0.7) (drill 0.4) (layers F.Cu B.Cu) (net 1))
 (via (at 107 117.5) (size 0.7) (drill 0.4) (layers F.Cu B.Cu) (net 1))
 (via (at 106 117.5) (size 0.7) (drill 0.4) (layers F.Cu B.Cu) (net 1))
 (via (at 105 117.5) (size 0.7) (drill 0.4) (layers F.Cu B.Cu) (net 1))
 (via (at 104 117.5) (size 0.7) (drill 0.4) (layers F.Cu B.Cu) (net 1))
 (via (at 103 117.5) (size 0.7) (drill 0.4) (layers F.Cu B.Cu) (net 1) (status 30))
 (via (at 100.5 114) (size 0.7) (drill 0.4) (layers F.Cu B.Cu) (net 1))
 (via (at 100.5 104) (size 0.7) (drill 0.4) (layers F.Cu B.Cu) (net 1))
 (via (at 104 100.5) (size 0.7) (drill 0.4) (layers F.Cu B.Cu) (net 1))
 (via (at 105 100.5) (size 0.7) (drill 0.4) (layers F.Cu B.Cu) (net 1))
 (via (at 106 100.5) (size 0.7) (drill 0.4) (layers F.Cu B.Cu) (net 1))
 (via (at 107 100.5) (size 0.7) (drill 0.4) (layers F.Cu B.Cu) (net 1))
 (via (at 108 100.5) (size 0.7) (drill 0.4) (layers F.Cu B.Cu) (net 1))
 (via (at 109 100.5) (size 0.7) (drill 0.4) (layers F.Cu B.Cu) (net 1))
 (via (at 110 100.5) (size 0.7) (drill 0.4) (layers F.Cu B.Cu) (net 1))
 (via (at 111 100.5) (size 0.7) (drill 0.4) (layers F.Cu B.Cu) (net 1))
 (via (at 112 100.5) (size 0.7) (drill 0.4) (layers F.Cu B.Cu) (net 1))
 (via (at 113 100.5) (size 0.7) (drill 0.4) (layers F.Cu B.Cu) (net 1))
 (via (at 114 100.5) (size 0.7) (drill 0.4) (layers F.Cu B.Cu) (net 1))
 (via (at 115 100.5) (size 0.7) (drill 0.4) (layers F.Cu B.Cu) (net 1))
 (via (at 116 100.5) (size 0.7) (drill 0.4) (layers F.Cu B.Cu) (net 1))
 (via (at 117 100.5) (size 0.7) (drill 0.4) (layers F.Cu B.Cu) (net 1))
 (via (at 118 100.5) (size 0.7) (drill 0.4) (layers F.Cu B.Cu) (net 1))
 (via (at 119 100.5) (size 0.7) (drill 0.4) (layers F.Cu B.Cu) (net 1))
 (via (at 120 100.5) (size 0.7) (drill 0.4) (layers F.Cu B.Cu) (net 1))
 (via (at 121 100.5) (size 0.7) (drill 0.4) (layers F.Cu B.Cu) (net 1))
 (via (at 122 100.5) (size 0.7) (drill 0.4) (layers F.Cu B.Cu) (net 1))
 (via (at 123 100.5) (size 0.7) (drill 0.4) (layers F.Cu B.Cu) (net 1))
 (via (at 124 100.5) (size 0.7) (drill 0.4) (layers F.Cu B.Cu) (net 1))
 (via (at 125 100.5) (size 0.7) (drill 0.4) (layers F.Cu B.Cu) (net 1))
 (via (at 126 100.5) (size 0.7) (drill 0.4) (layers F.Cu B.Cu) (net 1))
 (via (at 127 100.5) (size 0.7) (drill 0.4) (layers F.Cu B.Cu) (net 1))
 (via (at 128 100.5) (size 0.7) (drill 0.4) (layers F.Cu B.Cu) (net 1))
 (via (at 131.5 104) (size 0.7) (drill 0.4) (layers F.Cu B.Cu) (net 1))
 (via (at 131.5 114) (size 0.7) (drill 0.4) (layers F.Cu B.Cu) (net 1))
 (via (at 100.5 105) (size 0.7) (drill 0.4) (layers F.Cu B.Cu) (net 1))
 (via (at 100.5 113) (size 0.7) (drill 0.4) (layers F.Cu B.Cu) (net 1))
 (via (at 131.5 113) (size 0.7) (drill 0.4) (layers F.Cu B.Cu) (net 1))
 (via (at 131.5 105) (size 0.7) (drill 0.4) (layers F.Cu B.Cu) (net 1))
 (segment (start 120.11 107.62) (end 120.955 107.62) (width 0.22) (layer F.Cu) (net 4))
 (segment (start 118.87 108.86) (end 120.11 107.62) (width 0.22) (layer F.Cu) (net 4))
 (segment (start 117.9 108.86) (end 118.87 108.86) (width 0.22) (layer F.Cu) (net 4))
 (segment (start 116.33 105.73) (end 115.36 105.73) (width 0.22) (layer F.Cu) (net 4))
 (segment (start 117.9 107.3) (end 116.33 105.73) (width 0.22) (layer F.Cu) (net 4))
 (segment (start 117.9 108.86) (end 117.9 107.3) (width 0.22) (layer F.Cu) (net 4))
 (segment (start 120.447 110.16) (end 120.955 110.668) (width 0.22) (layer F.Cu) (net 5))
 (segment (start 117.9 110.16) (end 120.447 110.16) (width 0.22) (layer F.Cu) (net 5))
 (segment (start 114.39 104.43) (end 114.299999 104.520001) (width 0.22) (layer F.Cu) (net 5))
 (segment (start 117.375 110.16) (end 117.9 110.16) (width 0.22) (layer F.Cu) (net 5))
 (segment (start 114.299999 107.084999) (end 117.375 110.16) (width 0.22) (layer F.Cu) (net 5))
 (segment (start 114.299999 104.520001) (end 114.299999 107.084999) (width 0.22) (layer F.Cu) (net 5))
 (segment (start 115.36 104.43) (end 114.39 104.43) (width 0.22) (layer F.Cu) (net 5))
 (segment (start 109.999 107.62) (end 109.017 107.62) (width 0.22) (layer F.Cu) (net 6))
 (segment (start 112.7 105.525) (end 110.605 107.62) (width 0.22) (layer F.Cu) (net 6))
 (segment (start 110.605 107.62) (end 109.999 107.62) (width 0.22) (layer F.Cu) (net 6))
 (segment (start 112.7 105.08) (end 112.7 105.525) (width 0.22) (layer F.Cu) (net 6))
 (segment (start 114.27 109.51) (end 113.112 110.668) (width 0.22) (layer F.Cu) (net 7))
 (segment (start 109.999 110.668) (end 109.017 110.668) (width 0.22) (layer F.Cu) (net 7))
 (segment (start 113.112 110.668) (end 109.999 110.668) (width 0.22) (layer F.Cu) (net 7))
 (segment (start 115.24 109.51) (end 114.27 109.51) (width 0.22) (layer F.Cu) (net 7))
 (segment (start 104.733 107.62) (end 105.715 107.62) (width 0.22) (layer F.Cu) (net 2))
 (segment (start 103.302 109) (end 104.682 107.62) (width 0.22) (layer F.Cu) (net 2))
 (segment (start 104.682 107.62) (end 104.733 107.62) (width 0.22) (layer F.Cu) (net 2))
 (segment (start 102.032 109) (end 103.302 109) (width 0.22) (layer F.Cu) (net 2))
 (segment (start 130 108.018) (end 130 109) (width 0.22) (layer F.Cu) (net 3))
 (segment (start 129.602 107.62) (end 130 108.018) (width 0.22) (layer F.Cu) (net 3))
 (segment (start 124.257 107.62) (end 129.602 107.62) (width 0.22) (layer F.Cu) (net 3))
 (segment (start 116.51 113.97) (end 114.732 112.192) (width 0.22) (layer F.Cu) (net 8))
 (segment (start 116.51 115.24) (end 116.51 113.97) (width 0.22) (layer F.Cu) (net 8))
 (segment (start 108.839998 112.192) (end 107.112 110.464002) (width 0.22) (layer F.Cu) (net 8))
 (segment (start 114.732 112.192) (end 108.839998 112.192) (width 0.22) (layer F.Cu) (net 8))
 (segment (start 108.035 109.144) (end 109.017 109.144) (width 0.22) (layer F.Cu) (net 8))
 (segment (start 107.112 110.067) (end 108.035 109.144) (width 0.22) (layer F.Cu) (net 8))
 (segment (start 107.112 110.464002) (end 107.112 110.067) (width 0.22) (layer F.Cu) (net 8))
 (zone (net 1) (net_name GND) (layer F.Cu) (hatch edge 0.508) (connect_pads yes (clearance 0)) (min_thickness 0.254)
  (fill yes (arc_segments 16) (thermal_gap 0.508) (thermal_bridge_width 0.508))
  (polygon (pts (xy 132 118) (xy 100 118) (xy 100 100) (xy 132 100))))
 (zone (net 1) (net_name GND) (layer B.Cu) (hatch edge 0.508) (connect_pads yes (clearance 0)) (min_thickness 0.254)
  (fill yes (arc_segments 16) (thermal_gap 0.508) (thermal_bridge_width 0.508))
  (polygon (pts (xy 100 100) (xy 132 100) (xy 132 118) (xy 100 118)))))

